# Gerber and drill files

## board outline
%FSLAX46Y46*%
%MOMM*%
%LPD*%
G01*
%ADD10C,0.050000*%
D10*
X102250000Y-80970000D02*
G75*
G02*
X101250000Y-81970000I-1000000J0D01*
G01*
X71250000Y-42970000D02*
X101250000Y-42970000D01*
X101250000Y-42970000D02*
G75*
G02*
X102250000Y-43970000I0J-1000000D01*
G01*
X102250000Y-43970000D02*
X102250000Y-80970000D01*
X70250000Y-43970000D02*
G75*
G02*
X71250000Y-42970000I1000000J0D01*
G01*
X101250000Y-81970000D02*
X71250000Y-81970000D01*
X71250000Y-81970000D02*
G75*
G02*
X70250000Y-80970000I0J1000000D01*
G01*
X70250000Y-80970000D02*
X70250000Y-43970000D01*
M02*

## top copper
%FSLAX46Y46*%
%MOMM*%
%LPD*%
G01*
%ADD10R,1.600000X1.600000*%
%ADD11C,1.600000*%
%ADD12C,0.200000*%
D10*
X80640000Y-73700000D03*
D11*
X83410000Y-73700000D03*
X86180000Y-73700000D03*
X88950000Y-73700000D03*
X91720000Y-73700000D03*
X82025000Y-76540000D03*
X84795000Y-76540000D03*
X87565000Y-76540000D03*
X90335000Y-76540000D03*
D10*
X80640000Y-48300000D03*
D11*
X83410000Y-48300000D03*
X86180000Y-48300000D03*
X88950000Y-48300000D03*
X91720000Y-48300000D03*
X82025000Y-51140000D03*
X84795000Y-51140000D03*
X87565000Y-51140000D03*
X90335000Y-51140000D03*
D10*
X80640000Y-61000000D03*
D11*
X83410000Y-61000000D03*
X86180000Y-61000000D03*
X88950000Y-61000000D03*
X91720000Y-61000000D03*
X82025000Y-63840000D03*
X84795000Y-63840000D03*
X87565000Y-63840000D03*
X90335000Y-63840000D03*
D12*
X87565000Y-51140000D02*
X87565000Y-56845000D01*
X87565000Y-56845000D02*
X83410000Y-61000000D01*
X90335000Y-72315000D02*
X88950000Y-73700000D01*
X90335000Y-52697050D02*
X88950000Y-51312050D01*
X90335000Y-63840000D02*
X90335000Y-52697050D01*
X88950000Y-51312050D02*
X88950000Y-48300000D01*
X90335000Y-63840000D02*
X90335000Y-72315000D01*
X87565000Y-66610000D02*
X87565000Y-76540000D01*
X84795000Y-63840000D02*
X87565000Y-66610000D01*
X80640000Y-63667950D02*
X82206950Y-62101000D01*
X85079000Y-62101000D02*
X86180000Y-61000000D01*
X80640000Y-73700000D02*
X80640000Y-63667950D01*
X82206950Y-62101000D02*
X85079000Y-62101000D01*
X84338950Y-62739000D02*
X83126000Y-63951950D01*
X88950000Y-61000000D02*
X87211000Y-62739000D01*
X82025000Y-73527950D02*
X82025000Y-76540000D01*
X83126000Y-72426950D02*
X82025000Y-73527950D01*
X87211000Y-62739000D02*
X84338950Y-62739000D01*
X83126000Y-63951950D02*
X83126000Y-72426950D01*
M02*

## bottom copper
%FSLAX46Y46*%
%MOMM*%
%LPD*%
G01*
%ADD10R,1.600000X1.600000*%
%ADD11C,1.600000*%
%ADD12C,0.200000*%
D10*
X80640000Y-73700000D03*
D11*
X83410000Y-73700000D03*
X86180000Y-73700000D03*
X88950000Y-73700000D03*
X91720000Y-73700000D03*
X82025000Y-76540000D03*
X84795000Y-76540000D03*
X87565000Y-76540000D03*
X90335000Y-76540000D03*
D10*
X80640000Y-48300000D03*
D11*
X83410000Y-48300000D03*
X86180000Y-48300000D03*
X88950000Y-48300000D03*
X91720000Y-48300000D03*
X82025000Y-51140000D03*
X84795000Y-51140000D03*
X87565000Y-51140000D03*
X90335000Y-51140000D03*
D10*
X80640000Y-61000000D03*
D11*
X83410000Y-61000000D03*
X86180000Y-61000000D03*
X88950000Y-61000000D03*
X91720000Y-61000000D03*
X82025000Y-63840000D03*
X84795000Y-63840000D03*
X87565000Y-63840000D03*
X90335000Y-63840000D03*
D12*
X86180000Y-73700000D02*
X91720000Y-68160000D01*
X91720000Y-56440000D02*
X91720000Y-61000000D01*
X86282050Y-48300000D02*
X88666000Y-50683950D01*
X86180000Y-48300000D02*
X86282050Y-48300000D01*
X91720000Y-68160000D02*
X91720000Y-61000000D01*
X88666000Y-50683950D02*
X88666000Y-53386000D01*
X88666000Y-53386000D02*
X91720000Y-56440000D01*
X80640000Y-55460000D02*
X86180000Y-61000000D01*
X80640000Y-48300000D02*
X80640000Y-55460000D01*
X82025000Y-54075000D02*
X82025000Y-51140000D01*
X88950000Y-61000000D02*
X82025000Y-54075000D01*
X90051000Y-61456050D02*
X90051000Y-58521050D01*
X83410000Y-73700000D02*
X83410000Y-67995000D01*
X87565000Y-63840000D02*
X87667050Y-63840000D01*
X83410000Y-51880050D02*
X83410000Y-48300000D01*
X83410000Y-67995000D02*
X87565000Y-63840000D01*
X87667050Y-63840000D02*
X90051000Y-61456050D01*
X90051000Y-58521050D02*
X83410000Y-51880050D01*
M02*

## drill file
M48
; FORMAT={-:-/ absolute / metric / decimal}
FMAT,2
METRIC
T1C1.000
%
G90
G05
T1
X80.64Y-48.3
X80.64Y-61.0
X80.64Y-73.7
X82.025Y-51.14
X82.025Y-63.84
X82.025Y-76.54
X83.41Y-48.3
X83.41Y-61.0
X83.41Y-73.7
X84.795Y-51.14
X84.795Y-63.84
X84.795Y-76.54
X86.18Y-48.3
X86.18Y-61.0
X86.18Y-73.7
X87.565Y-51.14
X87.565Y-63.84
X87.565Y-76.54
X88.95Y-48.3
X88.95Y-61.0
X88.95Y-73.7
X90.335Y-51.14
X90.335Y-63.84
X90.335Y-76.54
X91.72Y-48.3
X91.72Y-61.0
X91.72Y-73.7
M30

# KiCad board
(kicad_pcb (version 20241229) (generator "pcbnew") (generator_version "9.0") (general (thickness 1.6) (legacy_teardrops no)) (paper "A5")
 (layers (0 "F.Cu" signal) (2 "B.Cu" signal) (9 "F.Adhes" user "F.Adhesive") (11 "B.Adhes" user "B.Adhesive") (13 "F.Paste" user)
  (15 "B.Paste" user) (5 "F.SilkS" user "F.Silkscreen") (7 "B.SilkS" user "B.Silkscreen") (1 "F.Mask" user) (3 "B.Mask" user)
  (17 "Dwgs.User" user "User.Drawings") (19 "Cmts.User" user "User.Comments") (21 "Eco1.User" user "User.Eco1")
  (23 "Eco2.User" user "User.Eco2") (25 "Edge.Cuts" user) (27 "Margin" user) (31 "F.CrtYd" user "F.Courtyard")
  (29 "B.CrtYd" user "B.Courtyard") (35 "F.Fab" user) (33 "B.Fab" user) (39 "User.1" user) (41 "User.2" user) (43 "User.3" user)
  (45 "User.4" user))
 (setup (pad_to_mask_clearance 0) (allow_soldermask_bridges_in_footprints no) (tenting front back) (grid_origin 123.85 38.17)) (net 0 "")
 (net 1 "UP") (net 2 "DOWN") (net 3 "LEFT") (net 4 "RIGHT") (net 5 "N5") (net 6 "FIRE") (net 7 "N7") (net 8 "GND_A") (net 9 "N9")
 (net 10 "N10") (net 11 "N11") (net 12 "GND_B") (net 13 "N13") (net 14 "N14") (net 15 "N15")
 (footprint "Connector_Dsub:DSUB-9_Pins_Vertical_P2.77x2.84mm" (layer "F.Cu") (at 80.64 73.7)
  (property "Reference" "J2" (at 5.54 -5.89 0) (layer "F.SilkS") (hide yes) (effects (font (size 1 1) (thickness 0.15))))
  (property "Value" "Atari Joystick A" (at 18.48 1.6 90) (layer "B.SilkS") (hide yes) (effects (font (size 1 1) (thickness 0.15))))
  (pad "1" thru_hole rect (at 0 0) (size 1.6 1.6) (drill 1) (layers "*.Cu" "*.Mask") (remove_unused_layers no) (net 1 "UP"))
  (pad "2" thru_hole circle (at 2.77 0) (size 1.6 1.6) (drill 1) (layers "*.Cu" "*.Mask") (remove_unused_layers no) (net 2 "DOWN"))
  (pad "3" thru_hole circle (at 5.54 0) (size 1.6 1.6) (drill 1) (layers "*.Cu" "*.Mask") (remove_unused_layers no) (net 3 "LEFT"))
  (pad "4" thru_hole circle (at 8.31 0) (size 1.6 1.6) (drill 1) (layers "*.Cu" "*.Mask") (remove_unused_layers no) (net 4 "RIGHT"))
  (pad "5" thru_hole circle (at 11.08 0) (size 1.6 1.6) (drill 1) (layers "*.Cu" "*.Mask") (remove_unused_layers no) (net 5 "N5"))
  (pad "6" thru_hole circle (at 1.385 2.84) (size 1.6 1.6) (drill 1) (layers "*.Cu" "*.Mask") (remove_unused_layers no) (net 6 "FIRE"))
  (pad "7" thru_hole circle (at 4.155 2.84) (size 1.6 1.6) (drill 1) (layers "*.Cu" "*.Mask") (remove_unused_layers no) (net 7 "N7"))
  (pad "8" thru_hole circle (at 6.925 2.84) (size 1.6 1.6) (drill 1) (layers "*.Cu" "*.Mask") (remove_unused_layers no) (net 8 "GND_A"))
  (pad "9" thru_hole circle (at 9.695 2.84) (size 1.6 1.6) (drill 1) (layers "*.Cu" "*.Mask") (remove_unused_layers no) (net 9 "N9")))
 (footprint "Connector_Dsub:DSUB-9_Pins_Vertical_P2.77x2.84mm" (layer "F.Cu") (at 80.64 48.3)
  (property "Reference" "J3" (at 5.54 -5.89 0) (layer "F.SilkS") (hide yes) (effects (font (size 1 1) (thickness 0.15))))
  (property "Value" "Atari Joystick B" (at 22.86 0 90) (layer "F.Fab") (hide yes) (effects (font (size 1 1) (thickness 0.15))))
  (pad "1" thru_hole rect (at 0 0) (size 1.6 1.6) (drill 1) (layers "*.Cu" "*.Mask") (remove_unused_layers no) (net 1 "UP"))
  (pad "2" thru_hole circle (at 2.77 0) (size 1.6 1.6) (drill 1) (layers "*.Cu" "*.Mask") (remove_unused_layers no) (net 2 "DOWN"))
  (pad "3" thru_hole circle (at 5.54 0) (size 1.6 1.6) (drill 1) (layers "*.Cu" "*.Mask") (remove_unused_layers no) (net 3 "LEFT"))
  (pad "4" thru_hole circle (at 8.31 0) (size 1.6 1.6) (drill 1) (layers "*.Cu" "*.Mask") (remove_unused_layers no) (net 4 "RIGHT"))
  (pad "5" thru_hole circle (at 11.08 0) (size 1.6 1.6) (drill 1) (layers "*.Cu" "*.Mask") (remove_unused_layers no) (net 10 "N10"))
  (pad "6" thru_hole circle (at 1.385 2.84) (size 1.6 1.6) (drill 1) (layers "*.Cu" "*.Mask") (remove_unused_layers no) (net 6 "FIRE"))
  (pad "7" thru_hole circle (at 4.155 2.84) (size 1.6 1.6) (drill 1) (layers "*.Cu" "*.Mask") (remove_unused_layers no) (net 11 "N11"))
  (pad "8" thru_hole circle (at 6.925 2.84) (size 1.6 1.6) (drill 1) (layers "*.Cu" "*.Mask") (remove_unused_layers no) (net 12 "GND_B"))
  (pad "9" thru_hole circle (at 9.695 2.84) (size 1.6 1.6) (drill 1) (layers "*.Cu" "*.Mask") (remove_unused_layers no) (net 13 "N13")))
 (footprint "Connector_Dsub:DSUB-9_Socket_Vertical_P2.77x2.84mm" (layer "B.Cu") (at 80.64 61 180)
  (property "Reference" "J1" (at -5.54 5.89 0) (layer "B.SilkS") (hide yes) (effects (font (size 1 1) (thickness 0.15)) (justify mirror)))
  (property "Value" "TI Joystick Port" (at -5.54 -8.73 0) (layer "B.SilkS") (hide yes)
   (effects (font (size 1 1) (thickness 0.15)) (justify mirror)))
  (pad "1" thru_hole rect (at 0 0 180) (size 1.6 1.6) (drill 1) (layers "*.Cu" "*.Mask") (remove_unused_layers no) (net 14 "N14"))
  (pad "2" thru_hole circle (at -2.77 0 180) (size 1.6 1.6) (drill 1) (layers "*.Cu" "*.Mask") (remove_unused_layers no) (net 12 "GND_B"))
  (pad "3" thru_hole circle (at -5.54 0 180) (size 1.6 1.6) (drill 1) (layers "*.Cu" "*.Mask") (remove_unused_layers no) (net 1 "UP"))
  (pad "4" thru_hole circle (at -8.31 0 180) (size 1.6 1.6) (drill 1) (layers "*.Cu" "*.Mask") (remove_unused_layers no) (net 6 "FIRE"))
  (pad "5" thru_hole circle (at -11.08 0 180) (size 1.6 1.6) (drill 1) (layers "*.Cu" "*.Mask") (remove_unused_layers no) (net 3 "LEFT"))
  (pad "6" thru_hole circle (at -1.385 -2.84 180) (size 1.6 1.6) (drill 1) (layers "*.Cu" "*.Mask") (remove_unused_layers no) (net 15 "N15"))
  (pad "7" thru_hole circle (at -4.155 -2.84 180) (size 1.6 1.6) (drill 1) (layers "*.Cu" "*.Mask") (remove_unused_layers no)
   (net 8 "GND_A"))
  (pad "8" thru_hole circle (at -6.925 -2.84 180) (size 1.6 1.6) (drill 1) (layers "*.Cu" "*.Mask") (remove_unused_layers no) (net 2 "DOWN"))
  (pad "9" thru_hole circle (at -9.695 -2.84 180) (size 1.6 1.6) (drill 1) (layers "*.Cu" "*.Mask") (remove_unused_layers no)
   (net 4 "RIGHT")))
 (gr_arc (start 102.25 80.97) (mid 101.957107 81.677107) (end 101.25 81.97) (stroke (width 0.05) (type default)) (layer "Edge.Cuts"))
 (gr_line (start 71.25 42.97) (end 101.25 42.97) (stroke (width 0.05) (type default)) (layer "Edge.Cuts"))
 (gr_arc (start 101.25 42.97) (mid 101.957107 43.262893) (end 102.25 43.97) (stroke (width 0.05) (type default)) (layer "Edge.Cuts"))
 (gr_line (start 102.25 43.97) (end 102.25 80.97) (stroke (width 0.05) (type default)) (layer "Edge.Cuts"))
 (gr_arc (start 70.25 43.97) (mid 70.542893 43.262893) (end 71.25 42.97) (stroke (width 0.05) (type default)) (layer "Edge.Cuts"))
 (gr_line (start 101.25 81.97) (end 71.25 81.97) (stroke (width 0.05) (type default)) (layer "Edge.Cuts"))
 (gr_arc (start 71.25 81.97) (mid 70.542893 81.677107) (end 70.25 80.97) (stroke (width 0.05) (type default)) (layer "Edge.Cuts"))
 (gr_line (start 70.25 80.97) (end 70.25 43.97) (stroke (width 0.05) (type default)) (layer "Edge.Cuts"))
 (segment (start 86.18 73.7) (end 91.72 68.16) (width 0.2) (layer "B.Cu") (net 3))
 (segment (start 91.72 56.44) (end 91.72 61) (width 0.2) (layer "B.Cu") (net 3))
 (segment (start 86.28205 48.3) (end 88.666 50.68395) (width 0.2) (layer "B.Cu") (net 3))
 (segment (start 86.18 48.3) (end 86.28205 48.3) (width 0.2) (layer "B.Cu") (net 3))
 (segment (start 91.72 68.16) (end 91.72 61) (width 0.2) (layer "B.Cu") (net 3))
 (segment (start 88.666 50.68395) (end 88.666 53.386) (width 0.2) (layer "B.Cu") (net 3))
 (segment (start 88.666 53.386) (end 91.72 56.44) (width 0.2) (layer "B.Cu") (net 3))
 (segment (start 87.565 51.14) (end 87.565 56.845) (width 0.2) (layer "F.Cu") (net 12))
 (segment (start 87.565 56.845) (end 83.41 61) (width 0.2) (layer "F.Cu") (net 12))
 (segment (start 90.335 72.315) (end 88.95 73.7) (width 0.2) (layer "F.Cu") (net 4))
 (segment (start 90.335 52.69705) (end 88.95 51.31205) (width 0.2) (layer "F.Cu") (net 4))
 (segment (start 90.335 63.84) (end 90.335 52.69705) (width 0.2) (layer "F.Cu") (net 4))
 (segment (start 88.95 51.31205) (end 88.95 48.3) (width 0.2) (layer "F.Cu") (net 4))
 (segment (start 90.335 63.84) (end 90.335 72.315) (width 0.2) (layer "F.Cu") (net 4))
 (segment (start 87.565 66.61) (end 87.565 76.54) (width 0.2) (layer "F.Cu") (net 8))
 (segment (start 84.795 63.84) (end 87.565 66.61) (width 0.2) (layer "F.Cu") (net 8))
 (segment (start 80.64 63.66795) (end 82.20695 62.101) (width 0.2) (layer "F.Cu") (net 1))
 (segment (start 85.079 62.101) (end 86.18 61) (width 0.2) (layer "F.Cu") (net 1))
 (segment (start 80.64 73.7) (end 80.64 63.66795) (width 0.2) (layer "F.Cu") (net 1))
 (segment (start 82.20695 62.101) (end 85.079 62.101) (width 0.2) (layer "F.Cu") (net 1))
 (segment (start 80.64 55.46) (end 86.18 61) (width 0.2) (layer "B.Cu") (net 1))
 (segment (start 80.64 48.3) (end 80.64 55.46) (width 0.2) (layer "B.Cu") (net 1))
 (segment (start 84.33895 62.739) (end 83.126 63.95195) (width 0.2) (layer "F.Cu") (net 6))
 (segment (start 88.95 61) (end 87.211 62.739) (width 0.2) (layer "F.Cu") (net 6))
 (segment (start 82.025 73.52795) (end 82.025 76.54) (width 0.2) (layer "F.Cu") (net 6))
 (segment (start 83.126 72.42695) (end 82.025 73.52795) (width 0.2) (layer "F.Cu") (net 6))
 (segment (start 87.211 62.739) (end 84.33895 62.739) (width 0.2) (layer "F.Cu") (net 6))
 (segment (start 83.126 63.95195) (end 83.126 72.42695) (width 0.2) (layer "F.Cu") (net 6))
 (segment (start 82.025 54.075) (end 82.025 51.14) (width 0.2) (layer "B.Cu") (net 6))
 (segment (start 88.95 61) (end 82.025 54.075) (width 0.2) (layer "B.Cu") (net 6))
 (segment (start 90.051 61.45605) (end 90.051 58.52105) (width 0.2) (layer "B.Cu") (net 2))
 (segment (start 83.41 73.7) (end 83.41 67.995) (width 0.2) (layer "B.Cu") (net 2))
 (segment (start 87.565 63.84) (end 87.66705 63.84) (width 0.2) (layer "B.Cu") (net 2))
 (segment (start 83.41 51.88005) (end 83.41 48.3) (width 0.2) (layer "B.Cu") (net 2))
 (segment (start 83.41 67.995) (end 87.565 63.84) (width 0.2) (layer "B.Cu") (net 2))
 (segment (start 87.66705 63.84) (end 90.051 61.45605) (width 0.2) (layer "B.Cu") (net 2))
 (segment (start 90.051 58.52105) (end 83.41 51.88005) (width 0.2) (layer "B.Cu") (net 2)))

